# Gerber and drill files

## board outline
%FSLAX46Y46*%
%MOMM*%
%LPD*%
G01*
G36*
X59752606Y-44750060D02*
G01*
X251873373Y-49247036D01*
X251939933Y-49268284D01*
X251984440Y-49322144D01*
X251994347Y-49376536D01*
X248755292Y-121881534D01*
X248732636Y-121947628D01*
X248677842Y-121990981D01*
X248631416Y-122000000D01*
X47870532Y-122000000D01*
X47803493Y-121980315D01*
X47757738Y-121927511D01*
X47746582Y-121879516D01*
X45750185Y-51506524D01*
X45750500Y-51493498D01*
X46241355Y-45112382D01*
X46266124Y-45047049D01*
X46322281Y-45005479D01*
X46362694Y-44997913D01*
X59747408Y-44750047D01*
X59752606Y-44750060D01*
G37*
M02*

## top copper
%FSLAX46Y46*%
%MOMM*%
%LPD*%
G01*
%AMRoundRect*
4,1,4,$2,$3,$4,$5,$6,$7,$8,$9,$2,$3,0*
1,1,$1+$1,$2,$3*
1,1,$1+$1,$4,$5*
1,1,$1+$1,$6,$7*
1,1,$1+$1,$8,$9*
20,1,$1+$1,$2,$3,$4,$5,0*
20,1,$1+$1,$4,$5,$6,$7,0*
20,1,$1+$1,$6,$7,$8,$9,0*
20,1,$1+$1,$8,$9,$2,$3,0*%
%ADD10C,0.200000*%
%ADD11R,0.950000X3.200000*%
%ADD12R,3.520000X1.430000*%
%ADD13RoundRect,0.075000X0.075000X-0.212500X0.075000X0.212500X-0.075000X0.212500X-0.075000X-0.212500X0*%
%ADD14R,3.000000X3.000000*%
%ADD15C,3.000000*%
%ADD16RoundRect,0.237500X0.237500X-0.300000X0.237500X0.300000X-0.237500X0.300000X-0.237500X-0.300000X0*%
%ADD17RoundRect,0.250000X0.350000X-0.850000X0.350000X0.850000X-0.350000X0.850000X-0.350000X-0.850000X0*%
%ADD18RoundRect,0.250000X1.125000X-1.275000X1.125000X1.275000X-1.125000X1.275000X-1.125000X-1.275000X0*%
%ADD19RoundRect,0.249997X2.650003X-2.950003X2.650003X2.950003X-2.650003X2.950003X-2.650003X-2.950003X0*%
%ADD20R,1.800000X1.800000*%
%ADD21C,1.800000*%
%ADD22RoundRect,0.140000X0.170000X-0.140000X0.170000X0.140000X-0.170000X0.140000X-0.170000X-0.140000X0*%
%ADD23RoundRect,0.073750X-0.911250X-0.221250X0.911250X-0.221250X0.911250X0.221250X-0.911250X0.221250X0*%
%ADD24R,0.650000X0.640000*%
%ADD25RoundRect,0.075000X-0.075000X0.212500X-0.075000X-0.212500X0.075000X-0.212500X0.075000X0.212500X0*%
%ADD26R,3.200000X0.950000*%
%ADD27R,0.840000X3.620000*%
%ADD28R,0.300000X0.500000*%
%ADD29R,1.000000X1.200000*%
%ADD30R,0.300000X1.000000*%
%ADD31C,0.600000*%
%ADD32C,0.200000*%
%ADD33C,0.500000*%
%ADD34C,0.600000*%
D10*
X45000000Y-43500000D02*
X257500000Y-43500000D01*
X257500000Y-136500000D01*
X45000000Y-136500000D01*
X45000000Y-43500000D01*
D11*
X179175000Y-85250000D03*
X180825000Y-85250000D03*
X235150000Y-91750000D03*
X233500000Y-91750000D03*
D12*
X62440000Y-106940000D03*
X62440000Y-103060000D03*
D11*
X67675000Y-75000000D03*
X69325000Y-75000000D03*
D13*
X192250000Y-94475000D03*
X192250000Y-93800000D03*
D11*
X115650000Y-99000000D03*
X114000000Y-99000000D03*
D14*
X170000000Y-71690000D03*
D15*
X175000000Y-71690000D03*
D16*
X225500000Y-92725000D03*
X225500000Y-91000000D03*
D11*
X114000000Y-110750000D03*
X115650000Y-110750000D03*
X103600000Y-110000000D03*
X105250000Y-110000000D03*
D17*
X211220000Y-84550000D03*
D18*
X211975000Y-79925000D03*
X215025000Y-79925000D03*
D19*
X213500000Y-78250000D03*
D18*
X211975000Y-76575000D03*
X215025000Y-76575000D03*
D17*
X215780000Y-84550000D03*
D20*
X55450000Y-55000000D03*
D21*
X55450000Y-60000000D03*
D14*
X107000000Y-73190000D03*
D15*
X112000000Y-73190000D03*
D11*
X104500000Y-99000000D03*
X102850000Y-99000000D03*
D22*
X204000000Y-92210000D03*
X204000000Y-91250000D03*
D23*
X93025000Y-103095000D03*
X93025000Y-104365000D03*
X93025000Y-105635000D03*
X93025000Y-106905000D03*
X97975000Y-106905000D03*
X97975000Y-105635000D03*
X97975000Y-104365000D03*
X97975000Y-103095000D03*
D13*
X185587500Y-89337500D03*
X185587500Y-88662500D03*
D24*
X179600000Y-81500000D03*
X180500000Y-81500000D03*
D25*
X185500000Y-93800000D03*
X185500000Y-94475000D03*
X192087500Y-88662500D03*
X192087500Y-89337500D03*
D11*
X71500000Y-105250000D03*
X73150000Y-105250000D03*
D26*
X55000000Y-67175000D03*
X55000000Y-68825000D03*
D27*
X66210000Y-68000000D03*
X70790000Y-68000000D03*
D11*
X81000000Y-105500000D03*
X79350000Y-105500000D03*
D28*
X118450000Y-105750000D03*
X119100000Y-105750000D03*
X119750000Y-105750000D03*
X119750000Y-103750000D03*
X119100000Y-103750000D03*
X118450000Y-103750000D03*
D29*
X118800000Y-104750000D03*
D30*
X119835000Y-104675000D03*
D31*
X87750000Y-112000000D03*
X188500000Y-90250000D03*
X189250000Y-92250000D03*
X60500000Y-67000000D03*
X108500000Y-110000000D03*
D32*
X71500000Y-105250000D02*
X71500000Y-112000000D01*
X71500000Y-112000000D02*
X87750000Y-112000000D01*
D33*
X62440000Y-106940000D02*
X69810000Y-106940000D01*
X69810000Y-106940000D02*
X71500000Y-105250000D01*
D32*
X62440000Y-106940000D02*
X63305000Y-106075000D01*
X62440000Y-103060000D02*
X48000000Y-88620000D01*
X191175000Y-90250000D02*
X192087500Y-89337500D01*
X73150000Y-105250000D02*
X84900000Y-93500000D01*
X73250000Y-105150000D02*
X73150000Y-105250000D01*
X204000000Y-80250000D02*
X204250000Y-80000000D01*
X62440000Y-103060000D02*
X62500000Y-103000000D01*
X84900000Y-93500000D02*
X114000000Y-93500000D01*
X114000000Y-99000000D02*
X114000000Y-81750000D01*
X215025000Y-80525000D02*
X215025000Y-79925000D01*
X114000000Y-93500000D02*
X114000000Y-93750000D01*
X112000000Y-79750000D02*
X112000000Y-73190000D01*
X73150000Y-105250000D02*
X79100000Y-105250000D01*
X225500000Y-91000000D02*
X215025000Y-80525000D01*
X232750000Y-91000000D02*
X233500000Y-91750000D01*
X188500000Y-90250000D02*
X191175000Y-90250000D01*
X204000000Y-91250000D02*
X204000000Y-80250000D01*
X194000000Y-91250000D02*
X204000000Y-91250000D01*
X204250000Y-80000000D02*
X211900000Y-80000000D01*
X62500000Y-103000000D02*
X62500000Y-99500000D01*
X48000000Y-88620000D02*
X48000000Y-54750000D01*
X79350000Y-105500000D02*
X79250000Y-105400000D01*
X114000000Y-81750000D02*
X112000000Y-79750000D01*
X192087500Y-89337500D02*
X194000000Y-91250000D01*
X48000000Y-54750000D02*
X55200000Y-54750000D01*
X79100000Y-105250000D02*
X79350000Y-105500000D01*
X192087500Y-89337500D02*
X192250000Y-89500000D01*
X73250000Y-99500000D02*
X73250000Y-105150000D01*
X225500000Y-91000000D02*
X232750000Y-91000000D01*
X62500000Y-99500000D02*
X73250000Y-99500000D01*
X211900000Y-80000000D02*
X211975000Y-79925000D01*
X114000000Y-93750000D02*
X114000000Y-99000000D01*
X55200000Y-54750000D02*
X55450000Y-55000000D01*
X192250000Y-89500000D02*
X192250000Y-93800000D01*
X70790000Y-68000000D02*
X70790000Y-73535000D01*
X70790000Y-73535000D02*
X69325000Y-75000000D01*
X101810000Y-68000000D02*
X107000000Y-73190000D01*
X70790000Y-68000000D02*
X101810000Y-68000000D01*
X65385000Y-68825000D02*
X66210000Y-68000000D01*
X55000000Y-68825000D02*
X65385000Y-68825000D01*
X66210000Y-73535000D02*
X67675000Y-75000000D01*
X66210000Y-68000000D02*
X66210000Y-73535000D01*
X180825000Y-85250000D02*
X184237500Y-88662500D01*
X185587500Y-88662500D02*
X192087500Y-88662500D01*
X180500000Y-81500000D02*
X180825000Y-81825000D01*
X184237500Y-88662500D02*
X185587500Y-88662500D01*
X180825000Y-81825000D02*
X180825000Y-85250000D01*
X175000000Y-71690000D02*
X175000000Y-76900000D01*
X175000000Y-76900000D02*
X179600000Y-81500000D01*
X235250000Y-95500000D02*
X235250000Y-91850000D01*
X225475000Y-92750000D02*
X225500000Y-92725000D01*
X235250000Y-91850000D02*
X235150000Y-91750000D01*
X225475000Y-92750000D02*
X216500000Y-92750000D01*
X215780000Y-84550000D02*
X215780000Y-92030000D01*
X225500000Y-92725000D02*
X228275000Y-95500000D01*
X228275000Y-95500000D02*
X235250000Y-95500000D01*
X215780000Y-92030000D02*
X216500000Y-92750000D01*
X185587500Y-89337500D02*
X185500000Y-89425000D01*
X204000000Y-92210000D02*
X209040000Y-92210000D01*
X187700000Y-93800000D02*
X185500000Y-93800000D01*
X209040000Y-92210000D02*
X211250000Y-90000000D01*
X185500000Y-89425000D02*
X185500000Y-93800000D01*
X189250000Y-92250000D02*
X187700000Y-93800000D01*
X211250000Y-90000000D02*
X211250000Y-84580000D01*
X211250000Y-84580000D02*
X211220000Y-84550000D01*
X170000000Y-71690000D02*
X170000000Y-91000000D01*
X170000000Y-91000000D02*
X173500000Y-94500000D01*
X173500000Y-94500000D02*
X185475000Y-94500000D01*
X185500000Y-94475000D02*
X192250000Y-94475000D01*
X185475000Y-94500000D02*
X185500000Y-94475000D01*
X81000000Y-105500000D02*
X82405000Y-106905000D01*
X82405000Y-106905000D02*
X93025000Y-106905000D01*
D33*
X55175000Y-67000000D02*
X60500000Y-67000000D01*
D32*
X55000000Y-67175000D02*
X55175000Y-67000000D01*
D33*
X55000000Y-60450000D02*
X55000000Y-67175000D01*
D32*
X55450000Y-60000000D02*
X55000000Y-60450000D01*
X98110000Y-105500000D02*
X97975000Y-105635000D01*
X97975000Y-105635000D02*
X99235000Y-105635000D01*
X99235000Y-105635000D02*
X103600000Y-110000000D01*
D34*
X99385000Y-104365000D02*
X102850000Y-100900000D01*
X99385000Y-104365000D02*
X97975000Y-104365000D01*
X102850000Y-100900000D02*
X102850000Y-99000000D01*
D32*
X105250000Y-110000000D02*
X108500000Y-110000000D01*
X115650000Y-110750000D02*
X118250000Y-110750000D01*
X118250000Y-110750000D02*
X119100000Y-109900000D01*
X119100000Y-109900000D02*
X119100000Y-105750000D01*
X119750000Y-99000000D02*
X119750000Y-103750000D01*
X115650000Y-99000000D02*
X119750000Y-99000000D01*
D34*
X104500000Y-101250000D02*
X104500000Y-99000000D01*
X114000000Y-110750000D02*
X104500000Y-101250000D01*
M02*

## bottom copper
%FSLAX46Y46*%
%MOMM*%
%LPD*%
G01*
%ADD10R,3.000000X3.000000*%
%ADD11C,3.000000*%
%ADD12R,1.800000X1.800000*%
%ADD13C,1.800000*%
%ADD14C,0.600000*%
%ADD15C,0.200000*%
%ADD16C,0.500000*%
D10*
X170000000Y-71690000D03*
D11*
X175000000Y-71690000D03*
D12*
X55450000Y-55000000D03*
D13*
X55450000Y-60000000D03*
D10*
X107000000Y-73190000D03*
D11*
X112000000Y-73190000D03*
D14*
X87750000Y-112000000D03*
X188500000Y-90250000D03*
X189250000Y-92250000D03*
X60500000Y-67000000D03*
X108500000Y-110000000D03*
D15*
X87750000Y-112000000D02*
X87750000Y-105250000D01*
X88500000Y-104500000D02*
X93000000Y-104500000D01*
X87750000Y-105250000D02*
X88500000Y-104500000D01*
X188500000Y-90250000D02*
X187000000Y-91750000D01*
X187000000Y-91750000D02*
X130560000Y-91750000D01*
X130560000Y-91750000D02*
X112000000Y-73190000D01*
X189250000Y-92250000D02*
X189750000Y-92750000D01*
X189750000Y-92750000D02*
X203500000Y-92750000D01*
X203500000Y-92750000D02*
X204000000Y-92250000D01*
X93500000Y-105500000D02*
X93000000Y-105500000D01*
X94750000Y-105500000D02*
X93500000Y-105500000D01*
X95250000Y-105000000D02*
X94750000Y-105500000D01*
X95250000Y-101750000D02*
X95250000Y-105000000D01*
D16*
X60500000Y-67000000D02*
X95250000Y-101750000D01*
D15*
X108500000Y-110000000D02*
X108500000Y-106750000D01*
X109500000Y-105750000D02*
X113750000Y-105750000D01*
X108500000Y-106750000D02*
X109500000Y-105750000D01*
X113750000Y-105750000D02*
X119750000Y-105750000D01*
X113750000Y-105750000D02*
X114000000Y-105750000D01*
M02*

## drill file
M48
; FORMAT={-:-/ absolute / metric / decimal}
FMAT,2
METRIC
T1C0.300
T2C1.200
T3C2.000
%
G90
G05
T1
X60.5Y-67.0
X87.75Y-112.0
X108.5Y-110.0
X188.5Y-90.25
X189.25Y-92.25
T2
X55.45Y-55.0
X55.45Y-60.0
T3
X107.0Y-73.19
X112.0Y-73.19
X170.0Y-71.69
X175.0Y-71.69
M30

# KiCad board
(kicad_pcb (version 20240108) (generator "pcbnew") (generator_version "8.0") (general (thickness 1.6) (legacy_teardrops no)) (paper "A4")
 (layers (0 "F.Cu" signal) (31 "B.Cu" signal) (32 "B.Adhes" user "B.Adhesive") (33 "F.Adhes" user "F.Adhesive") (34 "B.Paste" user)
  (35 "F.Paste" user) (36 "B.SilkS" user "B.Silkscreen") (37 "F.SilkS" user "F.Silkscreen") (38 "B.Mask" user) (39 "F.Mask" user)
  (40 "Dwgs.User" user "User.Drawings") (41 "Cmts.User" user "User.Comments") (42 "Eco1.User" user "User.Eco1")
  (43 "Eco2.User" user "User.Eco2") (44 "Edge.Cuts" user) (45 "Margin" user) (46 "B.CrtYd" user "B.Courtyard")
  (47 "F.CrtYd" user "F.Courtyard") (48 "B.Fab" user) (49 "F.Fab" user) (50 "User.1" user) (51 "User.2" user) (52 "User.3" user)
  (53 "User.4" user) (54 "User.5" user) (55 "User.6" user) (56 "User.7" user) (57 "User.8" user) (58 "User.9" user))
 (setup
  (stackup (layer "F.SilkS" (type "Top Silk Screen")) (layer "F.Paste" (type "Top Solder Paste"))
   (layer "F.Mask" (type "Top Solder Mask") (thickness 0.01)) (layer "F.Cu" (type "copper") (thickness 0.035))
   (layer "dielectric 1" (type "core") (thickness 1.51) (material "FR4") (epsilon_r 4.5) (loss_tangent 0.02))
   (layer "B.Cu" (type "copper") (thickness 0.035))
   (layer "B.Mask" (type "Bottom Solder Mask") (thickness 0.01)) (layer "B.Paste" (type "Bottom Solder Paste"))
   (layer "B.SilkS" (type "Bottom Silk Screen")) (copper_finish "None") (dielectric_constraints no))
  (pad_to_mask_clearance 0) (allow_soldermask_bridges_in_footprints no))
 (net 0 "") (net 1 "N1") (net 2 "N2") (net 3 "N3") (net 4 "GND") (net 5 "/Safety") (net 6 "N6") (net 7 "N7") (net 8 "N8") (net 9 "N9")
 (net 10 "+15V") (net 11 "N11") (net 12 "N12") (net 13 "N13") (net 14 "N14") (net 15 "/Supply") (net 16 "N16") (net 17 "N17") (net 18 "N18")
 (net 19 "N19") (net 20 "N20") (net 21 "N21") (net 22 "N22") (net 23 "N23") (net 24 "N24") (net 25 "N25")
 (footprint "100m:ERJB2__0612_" (layer "F.Cu") (at 180 85.25)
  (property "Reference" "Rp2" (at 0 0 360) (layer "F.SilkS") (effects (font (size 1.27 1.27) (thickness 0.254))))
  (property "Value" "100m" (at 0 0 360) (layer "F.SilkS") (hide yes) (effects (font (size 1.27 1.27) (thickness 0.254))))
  (pad "1" smd rect (at -0.825 0) (size 0.95 3.2) (layers "F.Cu" "F.Paste" "F.Mask") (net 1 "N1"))
  (pad "2" smd rect (at 0.825 0) (size 0.95 3.2) (layers "F.Cu" "F.Paste" "F.Mask") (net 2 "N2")))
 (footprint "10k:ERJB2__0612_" (layer "F.Cu") (at 234.325 91.75 180)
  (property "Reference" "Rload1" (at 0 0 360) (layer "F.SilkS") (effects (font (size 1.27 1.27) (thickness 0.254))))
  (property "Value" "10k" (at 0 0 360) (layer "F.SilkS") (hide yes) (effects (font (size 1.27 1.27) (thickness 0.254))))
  (pad "1" smd rect (at -0.825 0 180) (size 0.95 3.2) (layers "F.Cu" "F.Paste" "F.Mask") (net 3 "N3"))
  (pad "2" smd rect (at 0.825 0 180) (size 0.95 3.2) (layers "F.Cu" "F.Paste" "F.Mask") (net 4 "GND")))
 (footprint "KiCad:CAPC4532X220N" (layer "F.Cu") (at 62.44 105 90)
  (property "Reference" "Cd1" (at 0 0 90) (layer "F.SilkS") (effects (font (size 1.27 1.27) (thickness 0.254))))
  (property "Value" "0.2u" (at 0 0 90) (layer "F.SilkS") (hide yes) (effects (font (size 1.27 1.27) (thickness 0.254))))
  (pad "1" smd rect (at -1.94 0 90) (size 1.43 3.52) (layers "F.Cu" "F.Paste" "F.Mask") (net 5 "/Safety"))
  (pad "2" smd rect (at 1.94 0 90) (size 1.43 3.52) (layers "F.Cu" "F.Paste" "F.Mask") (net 4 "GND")))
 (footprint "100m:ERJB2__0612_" (layer "F.Cu") (at 68.5 75)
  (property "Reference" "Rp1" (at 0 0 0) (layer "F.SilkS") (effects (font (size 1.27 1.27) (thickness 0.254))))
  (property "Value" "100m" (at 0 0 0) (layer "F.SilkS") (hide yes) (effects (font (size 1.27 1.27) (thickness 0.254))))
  (pad "1" smd rect (at -0.825 0) (size 0.95 3.2) (layers "F.Cu" "F.Paste" "F.Mask") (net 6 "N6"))
  (pad "2" smd rect (at 0.825 0) (size 0.95 3.2) (layers "F.Cu" "F.Paste" "F.Mask") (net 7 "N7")))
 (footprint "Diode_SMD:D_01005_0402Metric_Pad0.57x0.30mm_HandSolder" (layer "F.Cu") (at 192.25 94.1375 90)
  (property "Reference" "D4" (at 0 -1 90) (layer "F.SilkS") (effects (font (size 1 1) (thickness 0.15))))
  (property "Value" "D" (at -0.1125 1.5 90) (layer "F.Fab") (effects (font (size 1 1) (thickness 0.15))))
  (pad "" smd roundrect (at -0.3625 0 90) (size 0.41 0.27) (layers "F.Paste") (roundrect_rratio 0.25))
  (pad "" smd roundrect (at 0.3625 0 90) (size 0.41 0.27) (layers "F.Paste") (roundrect_rratio 0.25))
  (pad "1" smd roundrect (at -0.3375 0 90) (size 0.575 0.3) (layers "F.Cu" "F.Mask") (roundrect_rratio 0.25) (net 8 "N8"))
  (pad "2" smd roundrect (at 0.3375 0 90) (size 0.575 0.3) (layers "F.Cu" "F.Mask") (roundrect_rratio 0.25) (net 4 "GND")))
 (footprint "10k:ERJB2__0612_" (layer "F.Cu") (at 114.825 99 180)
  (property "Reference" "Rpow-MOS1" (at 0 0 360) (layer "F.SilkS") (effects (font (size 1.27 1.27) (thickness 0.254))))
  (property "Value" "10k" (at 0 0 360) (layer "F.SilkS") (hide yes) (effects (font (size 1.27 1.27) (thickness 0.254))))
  (pad "1" smd rect (at -0.825 0 180) (size 0.95 3.2) (layers "F.Cu" "F.Paste" "F.Mask") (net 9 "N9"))
  (pad "2" smd rect (at 0.825 0 180) (size 0.95 3.2) (layers "F.Cu" "F.Paste" "F.Mask") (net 4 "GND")))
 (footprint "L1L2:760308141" (layer "F.Cu") (at 170 71.69)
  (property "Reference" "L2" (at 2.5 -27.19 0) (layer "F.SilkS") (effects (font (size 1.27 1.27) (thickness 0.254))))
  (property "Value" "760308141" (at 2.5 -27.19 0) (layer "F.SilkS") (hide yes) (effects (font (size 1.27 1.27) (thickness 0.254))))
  (pad "1" thru_hole rect (at 0 0) (size 3 3) (drill 2) (layers "*.Cu" "*.Mask") (remove_unused_layers no) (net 8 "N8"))
  (pad "2" thru_hole circle (at 5 0) (size 3 3) (drill 2) (layers "*.Cu" "*.Mask") (remove_unused_layers no) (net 1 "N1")))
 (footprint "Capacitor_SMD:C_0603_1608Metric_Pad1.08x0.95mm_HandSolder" (layer "F.Cu") (at 225.5 91.8625 90)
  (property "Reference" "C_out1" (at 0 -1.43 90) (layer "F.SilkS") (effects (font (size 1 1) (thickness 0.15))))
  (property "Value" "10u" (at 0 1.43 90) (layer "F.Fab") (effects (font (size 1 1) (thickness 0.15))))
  (pad "1" smd roundrect (at -0.8625 0 90) (size 1.075 0.95) (layers "F.Cu" "F.Paste" "F.Mask") (roundrect_rratio 0.25) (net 3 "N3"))
  (pad "2" smd roundrect (at 0.8625 0 90) (size 1.075 0.95) (layers "F.Cu" "F.Paste" "F.Mask") (roundrect_rratio 0.25) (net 4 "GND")))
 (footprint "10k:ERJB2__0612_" (layer "F.Cu") (at 114.825 110.75)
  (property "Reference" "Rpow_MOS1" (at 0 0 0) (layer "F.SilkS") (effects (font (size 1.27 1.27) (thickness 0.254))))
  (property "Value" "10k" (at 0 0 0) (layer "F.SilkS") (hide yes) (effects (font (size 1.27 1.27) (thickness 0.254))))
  (pad "1" smd rect (at -0.825 0) (size 0.95 3.2) (layers "F.Cu" "F.Paste" "F.Mask") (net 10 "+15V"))
  (pad "2" smd rect (at 0.825 0) (size 0.95 3.2) (layers "F.Cu" "F.Paste" "F.Mask") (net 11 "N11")))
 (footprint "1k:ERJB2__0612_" (layer "F.Cu") (at 104.425 110)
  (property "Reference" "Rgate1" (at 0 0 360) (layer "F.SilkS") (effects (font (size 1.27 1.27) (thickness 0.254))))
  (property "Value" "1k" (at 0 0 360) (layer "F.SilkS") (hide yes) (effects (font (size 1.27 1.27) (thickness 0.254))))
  (pad "1" smd rect (at -0.825 0) (size 0.95 3.2) (layers "F.Cu" "F.Paste" "F.Mask") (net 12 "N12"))
  (pad "2" smd rect (at 0.825 0) (size 0.95 3.2) (layers "F.Cu" "F.Paste" "F.Mask") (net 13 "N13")))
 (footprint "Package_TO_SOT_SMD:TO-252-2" (layer "F.Cu") (at 213.5 79.51 90)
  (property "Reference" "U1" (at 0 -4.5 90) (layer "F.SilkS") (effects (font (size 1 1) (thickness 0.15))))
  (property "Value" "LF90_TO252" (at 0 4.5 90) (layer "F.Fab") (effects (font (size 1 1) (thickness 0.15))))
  (pad "1" smd roundrect (at -5.04 -2.28 90) (size 2.2 1.2) (layers "F.Cu" "F.Paste" "F.Mask") (roundrect_rratio 0.208333) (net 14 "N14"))
  (pad "2" smd roundrect (at -0.415 -1.525 90) (size 3.05 2.75) (layers "F.Cu" "F.Paste") (roundrect_rratio 0.090909) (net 4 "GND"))
  (pad "2" smd roundrect (at -0.415 1.525 90) (size 3.05 2.75) (layers "F.Cu" "F.Paste") (roundrect_rratio 0.090909) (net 4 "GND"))
  (pad "2" smd roundrect (at 1.26 0 90) (size 6.4 5.8) (layers "F.Cu" "F.Mask") (roundrect_rratio 0.043103) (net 4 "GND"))
  (pad "2" smd roundrect (at 2.935 -1.525 90) (size 3.05 2.75) (layers "F.Cu" "F.Paste") (roundrect_rratio 0.090909) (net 4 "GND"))
  (pad "2" smd roundrect (at 2.935 1.525 90) (size 3.05 2.75) (layers "F.Cu" "F.Paste") (roundrect_rratio 0.090909) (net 4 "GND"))
  (pad "3" smd roundrect (at -5.04 2.28 90) (size 2.2 1.2) (layers "F.Cu" "F.Paste" "F.Mask") (roundrect_rratio 0.208333) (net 3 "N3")))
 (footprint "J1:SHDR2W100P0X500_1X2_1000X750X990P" (layer "F.Cu") (at 55.45 55 -90)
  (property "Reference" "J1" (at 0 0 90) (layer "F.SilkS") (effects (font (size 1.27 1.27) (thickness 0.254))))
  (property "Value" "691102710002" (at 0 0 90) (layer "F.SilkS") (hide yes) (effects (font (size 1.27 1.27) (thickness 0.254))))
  (pad "1" thru_hole rect (at 0 0 270) (size 1.8 1.8) (drill 1.2) (layers "*.Cu" "*.Mask") (remove_unused_layers no) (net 4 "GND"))
  (pad "2" thru_hole circle (at 5 0 270) (size 1.8 1.8) (drill 1.2) (layers "*.Cu" "*.Mask") (remove_unused_layers no) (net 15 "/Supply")))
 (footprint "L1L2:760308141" (layer "F.Cu") (at 107 73.19)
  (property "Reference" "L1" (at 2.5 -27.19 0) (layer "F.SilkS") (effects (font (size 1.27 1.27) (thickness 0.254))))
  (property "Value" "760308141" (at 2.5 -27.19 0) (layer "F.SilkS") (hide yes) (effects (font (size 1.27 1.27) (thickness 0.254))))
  (pad "1" thru_hole rect (at 0 0) (size 3 3) (drill 2) (layers "*.Cu" "*.Mask") (remove_unused_layers no) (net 7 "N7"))
  (pad "2" thru_hole circle (at 5 0) (size 3 3) (drill 2) (layers "*.Cu" "*.Mask") (remove_unused_layers no) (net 4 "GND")))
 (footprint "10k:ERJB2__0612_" (layer "F.Cu") (at 103.675 99 180)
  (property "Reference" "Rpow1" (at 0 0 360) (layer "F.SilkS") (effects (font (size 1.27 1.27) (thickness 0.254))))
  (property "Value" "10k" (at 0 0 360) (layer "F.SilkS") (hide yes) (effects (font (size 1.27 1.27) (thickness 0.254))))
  (pad "1" smd rect (at -0.825 0 180) (size 0.95 3.2) (layers "F.Cu" "F.Paste" "F.Mask") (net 10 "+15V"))
  (pad "2" smd rect (at 0.825 0 180) (size 0.95 3.2) (layers "F.Cu" "F.Paste" "F.Mask") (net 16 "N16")))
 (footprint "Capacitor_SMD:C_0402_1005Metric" (layer "F.Cu") (at 204 91.73 90)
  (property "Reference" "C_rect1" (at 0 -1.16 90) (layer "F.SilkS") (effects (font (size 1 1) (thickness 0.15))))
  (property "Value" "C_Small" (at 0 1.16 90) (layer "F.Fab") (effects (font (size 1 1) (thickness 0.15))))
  (pad "1" smd roundrect (at -0.48 0 90) (size 0.56 0.62) (layers "F.Cu" "F.Paste" "F.Mask") (roundrect_rratio 0.25) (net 14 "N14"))
  (pad "2" smd roundrect (at 0.48 0 90) (size 0.56 0.62) (layers "F.Cu" "F.Paste" "F.Mask") (roundrect_rratio 0.25) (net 4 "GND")))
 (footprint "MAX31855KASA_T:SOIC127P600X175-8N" (layer "F.Cu") (at 95.5 105)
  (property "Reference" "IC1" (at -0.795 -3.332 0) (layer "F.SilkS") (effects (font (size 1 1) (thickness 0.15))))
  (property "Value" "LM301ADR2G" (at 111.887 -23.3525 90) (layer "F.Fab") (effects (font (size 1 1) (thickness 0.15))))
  (pad "1" smd roundrect (at -2.475 -1.905) (size 1.97 0.59) (layers "F.Cu" "F.Paste" "F.Mask") (roundrect_rratio 0.125) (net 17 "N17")
   (solder_mask_margin 0.102))
  (pad "2" smd roundrect (at -2.475 -0.635) (size 1.97 0.59) (layers "F.Cu" "F.Paste" "F.Mask") (roundrect_rratio 0.125) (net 5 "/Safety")
   (solder_mask_margin 0.102))
  (pad "3" smd roundrect (at -2.475 0.635) (size 1.97 0.59) (layers "F.Cu" "F.Paste" "F.Mask") (roundrect_rratio 0.125) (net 15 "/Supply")
   (solder_mask_margin 0.102))
  (pad "4" smd roundrect (at -2.475 1.905) (size 1.97 0.59) (layers "F.Cu" "F.Paste" "F.Mask") (roundrect_rratio 0.125) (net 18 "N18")
   (solder_mask_margin 0.102))
  (pad "5" smd roundrect (at 2.475 1.905) (size 1.97 0.59) (layers "F.Cu" "F.Paste" "F.Mask") (roundrect_rratio 0.125) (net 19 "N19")
   (solder_mask_margin 0.102))
  (pad "6" smd roundrect (at 2.475 0.635) (size 1.97 0.59) (layers "F.Cu" "F.Paste" "F.Mask") (roundrect_rratio 0.125) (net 12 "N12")
   (solder_mask_margin 0.102))
  (pad "7" smd roundrect (at 2.475 -0.635) (size 1.97 0.59) (layers "F.Cu" "F.Paste" "F.Mask") (roundrect_rratio 0.125) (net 16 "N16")
   (solder_mask_margin 0.102))
  (pad "8" smd roundrect (at 2.475 -1.905) (size 1.97 0.59) (layers "F.Cu" "F.Paste" "F.Mask") (roundrect_rratio 0.125) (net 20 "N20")
   (solder_mask_margin 0.102)))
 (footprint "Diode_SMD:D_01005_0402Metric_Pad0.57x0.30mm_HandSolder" (layer "F.Cu") (at 185.5875 89 90)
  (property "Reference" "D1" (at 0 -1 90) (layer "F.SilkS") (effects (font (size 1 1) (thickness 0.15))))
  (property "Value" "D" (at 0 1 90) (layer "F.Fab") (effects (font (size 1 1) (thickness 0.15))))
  (pad "" smd roundrect (at -0.3625 0 90) (size 0.41 0.27) (layers "F.Paste") (roundrect_rratio 0.25))
  (pad "" smd roundrect (at 0.3625 0 90) (size 0.41 0.27) (layers "F.Paste") (roundrect_rratio 0.25))
  (pad "1" smd roundrect (at -0.3375 0 90) (size 0.575 0.3) (layers "F.Cu" "F.Mask") (roundrect_rratio 0.25) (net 14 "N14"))
  (pad "2" smd roundrect (at 0.3375 0 90) (size 0.575 0.3) (layers "F.Cu" "F.Mask") (roundrect_rratio 0.25) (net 2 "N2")))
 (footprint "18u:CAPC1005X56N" (layer "F.Cu") (at 180.05 81.5)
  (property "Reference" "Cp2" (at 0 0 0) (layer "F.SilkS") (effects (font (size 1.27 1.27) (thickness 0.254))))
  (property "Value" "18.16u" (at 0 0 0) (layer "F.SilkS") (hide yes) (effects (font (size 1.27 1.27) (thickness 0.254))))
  (pad "1" smd rect (at -0.45 0 90) (size 0.64 0.65) (layers "F.Cu" "F.Paste" "F.Mask") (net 1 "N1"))
  (pad "2" smd rect (at 0.45 0 90) (size 0.64 0.65) (layers "F.Cu" "F.Paste" "F.Mask") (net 2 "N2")))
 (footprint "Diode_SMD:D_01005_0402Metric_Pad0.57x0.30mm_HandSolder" (layer "F.Cu") (at 185.5 94.1375 -90)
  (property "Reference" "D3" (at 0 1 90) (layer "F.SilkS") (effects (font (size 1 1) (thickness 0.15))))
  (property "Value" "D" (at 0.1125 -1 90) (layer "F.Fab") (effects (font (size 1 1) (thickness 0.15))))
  (pad "" smd roundrect (at -0.3625 0 270) (size 0.41 0.27) (layers "F.Paste") (roundrect_rratio 0.25))
  (pad "" smd roundrect (at 0.3625 0 270) (size 0.41 0.27) (layers "F.Paste") (roundrect_rratio 0.25))
  (pad "1" smd roundrect (at -0.3375 0 270) (size 0.575 0.3) (layers "F.Cu" "F.Mask") (roundrect_rratio 0.25) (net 14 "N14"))
  (pad "2" smd roundrect (at 0.3375 0 270) (size 0.575 0.3) (layers "F.Cu" "F.Mask") (roundrect_rratio 0.25) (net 8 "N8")))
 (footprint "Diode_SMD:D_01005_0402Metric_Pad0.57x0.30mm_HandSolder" (layer "F.Cu") (at 192.0875 89 -90)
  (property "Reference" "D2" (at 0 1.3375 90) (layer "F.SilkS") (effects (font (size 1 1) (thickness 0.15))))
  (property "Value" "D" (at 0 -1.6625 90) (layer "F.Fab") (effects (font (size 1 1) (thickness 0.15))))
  (pad "" smd roundrect (at -0.3625 0 270) (size 0.41 0.27) (layers "F.Paste") (roundrect_rratio 0.25))
  (pad "" smd roundrect (at 0.3625 0 270) (size 0.41 0.27) (layers "F.Paste") (roundrect_rratio 0.25))
  (pad "1" smd roundrect (at -0.3375 0 270) (size 0.575 0.3) (layers "F.Cu" "F.Mask") (roundrect_rratio 0.25) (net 2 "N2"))
  (pad "2" smd roundrect (at 0.3375 0 270) (size 0.575 0.3) (layers "F.Cu" "F.Mask") (roundrect_rratio 0.25) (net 4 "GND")))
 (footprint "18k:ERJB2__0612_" (layer "F.Cu") (at 72.325 105.25)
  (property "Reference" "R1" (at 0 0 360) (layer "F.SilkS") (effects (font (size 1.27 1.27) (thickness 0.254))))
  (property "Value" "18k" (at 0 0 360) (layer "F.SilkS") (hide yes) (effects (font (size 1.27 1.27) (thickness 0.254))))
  (pad "1" smd rect (at -0.825 0) (size 0.95 3.2) (layers "F.Cu" "F.Paste" "F.Mask") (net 5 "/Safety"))
  (pad "2" smd rect (at 0.825 0) (size 0.95 3.2) (layers "F.Cu" "F.Paste" "F.Mask") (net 4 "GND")))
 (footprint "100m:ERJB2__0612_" (layer "F.Cu") (at 55 68 -90)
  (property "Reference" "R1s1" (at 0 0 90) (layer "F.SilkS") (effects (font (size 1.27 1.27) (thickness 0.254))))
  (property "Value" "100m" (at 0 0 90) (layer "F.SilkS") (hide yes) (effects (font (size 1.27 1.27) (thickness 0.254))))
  (pad "1" smd rect (at -0.825 0 270) (size 0.95 3.2) (layers "F.Cu" "F.Paste" "F.Mask") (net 15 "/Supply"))
  (pad "2" smd rect (at 0.825 0 270) (size 0.95 3.2) (layers "F.Cu" "F.Paste" "F.Mask") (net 6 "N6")))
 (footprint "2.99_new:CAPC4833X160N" (layer "F.Cu") (at 68.5 68)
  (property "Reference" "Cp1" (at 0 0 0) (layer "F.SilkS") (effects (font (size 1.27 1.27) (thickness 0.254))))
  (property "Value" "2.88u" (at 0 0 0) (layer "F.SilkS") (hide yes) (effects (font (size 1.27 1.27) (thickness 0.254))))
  (pad "1" smd rect (at -2.29 0) (size 0.84 3.62) (layers "F.Cu" "F.Paste" "F.Mask") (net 6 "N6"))
  (pad "2" smd rect (at 2.29 0) (size 0.84 3.62) (layers "F.Cu" "F.Paste" "F.Mask") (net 7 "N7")))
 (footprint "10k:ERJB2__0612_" (layer "F.Cu") (at 80.175 105.5 180)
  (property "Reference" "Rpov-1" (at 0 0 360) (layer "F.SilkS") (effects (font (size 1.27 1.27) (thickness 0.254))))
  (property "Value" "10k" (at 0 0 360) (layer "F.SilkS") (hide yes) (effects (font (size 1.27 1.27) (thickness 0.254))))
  (pad "1" smd rect (at -0.825 0 180) (size 0.95 3.2) (layers "F.Cu" "F.Paste" "F.Mask") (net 18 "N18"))
  (pad "2" smd rect (at 0.825 0 180) (size 0.95 3.2) (layers "F.Cu" "F.Paste" "F.Mask") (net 4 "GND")))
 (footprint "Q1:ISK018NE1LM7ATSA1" (layer "F.Cu") (at 119.1 104.75)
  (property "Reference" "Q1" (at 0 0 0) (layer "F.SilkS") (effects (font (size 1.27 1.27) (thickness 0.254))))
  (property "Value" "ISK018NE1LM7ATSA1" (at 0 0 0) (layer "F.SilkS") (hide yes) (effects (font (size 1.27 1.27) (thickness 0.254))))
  (pad "1" smd rect (at -0.65 1) (size 0.3 0.5) (layers "F.Cu" "F.Paste" "F.Mask") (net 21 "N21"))
  (pad "2" smd rect (at 0 1) (size 0.3 0.5) (layers "F.Cu" "F.Paste" "F.Mask") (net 11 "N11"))
  (pad "3" smd rect (at 0.65 1) (size 0.3 0.5) (layers "F.Cu" "F.Paste" "F.Mask") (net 13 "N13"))
  (pad "4" smd rect (at 0.65 -1) (size 0.3 0.5) (layers "F.Cu" "F.Paste" "F.Mask") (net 9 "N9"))
  (pad "5" smd rect (at 0 -1) (size 0.3 0.5) (layers "F.Cu" "F.Paste" "F.Mask") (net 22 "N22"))
  (pad "6" smd rect (at -0.65 -1) (size 0.3 0.5) (layers "F.Cu" "F.Paste" "F.Mask") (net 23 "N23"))
  (pad "7" smd rect (at -0.3 0) (size 1 1.2) (layers "F.Cu" "F.Paste" "F.Mask") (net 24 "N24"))
  (pad "8" smd rect (at 0.735 -0.075) (size 0.3 1) (layers "F.Cu" "F.Paste" "F.Mask") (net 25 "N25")))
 (gr_rect (start 45 43.5) (end 257.5 136.5) (stroke (width 0.2) (type default)) (fill none) (layer "F.Cu"))
 (segment (start 71.5 105.25) (end 71.5 112) (width 0.2) (layer "F.Cu") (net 5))
 (segment (start 71.5 112) (end 87.75 112) (width 0.2) (layer "F.Cu") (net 5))
 (segment (start 62.44 106.94) (end 69.81 106.94) (width 0.5) (layer "F.Cu") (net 5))
 (segment (start 69.81 106.94) (end 71.5 105.25) (width 0.5) (layer "F.Cu") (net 5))
 (segment (start 62.44 106.94) (end 63.305 106.075) (width 0.2) (layer "F.Cu") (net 5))
 (via (at 87.75 112) (size 0.6) (drill 0.3) (layers "F.Cu" "B.Cu") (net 5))
 (segment (start 87.75 112) (end 87.75 105.25) (width 0.2) (layer "B.Cu") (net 5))
 (segment (start 88.5 104.5) (end 93 104.5) (width 0.2) (layer "B.Cu") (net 5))
 (segment (start 87.75 105.25) (end 88.5 104.5) (width 0.2) (layer "B.Cu") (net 5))
 (segment (start 62.44 103.06) (end 48 88.62) (width 0.2) (layer "F.Cu") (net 4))
 (segment (start 191.175 90.25) (end 192.0875 89.3375) (width 0.2) (layer "F.Cu") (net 4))
 (segment (start 73.15 105.25) (end 84.9 93.5) (width 0.2) (layer "F.Cu") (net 4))
 (segment (start 73.25 105.15) (end 73.15 105.25) (width 0.2) (layer "F.Cu") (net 4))
 (segment (start 204 80.25) (end 204.25 80) (width 0.2) (layer "F.Cu") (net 4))
 (segment (start 62.44 103.06) (end 62.5 103) (width 0.2) (layer "F.Cu") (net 4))
 (segment (start 84.9 93.5) (end 114 93.5) (width 0.2) (layer "F.Cu") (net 4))
 (segment (start 114 99) (end 114 81.75) (width 0.2) (layer "F.Cu") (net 4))
 (segment (start 215.025 80.525) (end 215.025 79.925) (width 0.2) (layer "F.Cu") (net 4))
 (segment (start 114 93.5) (end 114 93.75) (width 0.2) (layer "F.Cu") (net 4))
 (segment (start 112 79.75) (end 112 73.19) (width 0.2) (layer "F.Cu") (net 4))
 (segment (start 73.15 105.25) (end 79.1 105.25) (width 0.2) (layer "F.Cu") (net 4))
 (segment (start 225.5 91) (end 215.025 80.525) (width 0.2) (layer "F.Cu") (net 4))
 (segment (start 232.75 91) (end 233.5 91.75) (width 0.2) (layer "F.Cu") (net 4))
 (segment (start 188.5 90.25) (end 191.175 90.25) (width 0.2) (layer "F.Cu") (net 4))
 (segment (start 204 91.25) (end 204 80.25) (width 0.2) (layer "F.Cu") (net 4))
 (segment (start 194 91.25) (end 204 91.25) (width 0.2) (layer "F.Cu") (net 4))
 (segment (start 204.25 80) (end 211.9 80) (width 0.2) (layer "F.Cu") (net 4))
 (segment (start 62.5 103) (end 62.5 99.5) (width 0.2) (layer "F.Cu") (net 4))
 (segment (start 48 88.62) (end 48 54.75) (width 0.2) (layer "F.Cu") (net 4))
 (segment (start 79.35 105.5) (end 79.25 105.4) (width 0.2) (layer "F.Cu") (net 4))
 (segment (start 114 81.75) (end 112 79.75) (width 0.2) (layer "F.Cu") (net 4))
 (segment (start 192.0875 89.3375) (end 194 91.25) (width 0.2) (layer "F.Cu") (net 4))
 (segment (start 48 54.75) (end 55.2 54.75) (width 0.2) (layer "F.Cu") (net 4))
 (segment (start 79.1 105.25) (end 79.35 105.5) (width 0.2) (layer "F.Cu") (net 4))
 (segment (start 192.0875 89.3375) (end 192.25 89.5) (width 0.2) (layer "F.Cu") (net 4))
 (segment (start 73.25 99.5) (end 73.25 105.15) (width 0.2) (layer "F.Cu") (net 4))
 (segment (start 225.5 91) (end 232.75 91) (width 0.2) (layer "F.Cu") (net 4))
 (segment (start 62.5 99.5) (end 73.25 99.5) (width 0.2) (layer "F.Cu") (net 4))
 (segment (start 211.9 80) (end 211.975 79.925) (width 0.2) (layer "F.Cu") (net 4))
 (segment (start 114 93.75) (end 114 99) (width 0.2) (layer "F.Cu") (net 4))
 (segment (start 55.2 54.75) (end 55.45 55) (width 0.2) (layer "F.Cu") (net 4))
 (segment (start 192.25 89.5) (end 192.25 93.8) (width 0.2) (layer "F.Cu") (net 4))
 (via (at 188.5 90.25) (size 0.6) (drill 0.3) (layers "F.Cu" "B.Cu") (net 4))
 (segment (start 188.5 90.25) (end 187 91.75) (width 0.2) (layer "B.Cu") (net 4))
 (segment (start 187 91.75) (end 130.56 91.75) (width 0.2) (layer "B.Cu") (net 4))
 (segment (start 130.56 91.75) (end 112 73.19) (width 0.2) (layer "B.Cu") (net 4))
 (segment (start 70.79 68) (end 70.79 73.535) (width 0.2) (layer "F.Cu") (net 7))
 (segment (start 70.79 73.535) (end 69.325 75) (width 0.2) (layer "F.Cu") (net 7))
 (segment (start 101.81 68) (end 107 73.19) (width 0.2) (layer "F.Cu") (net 7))
 (segment (start 70.79 68) (end 101.81 68) (width 0.2) (layer "F.Cu") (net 7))
 (segment (start 65.385 68.825) (end 66.21 68) (width 0.2) (layer "F.Cu") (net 6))
 (segment (start 55 68.825) (end 65.385 68.825) (width 0.2) (layer "F.Cu") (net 6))
 (segment (start 66.21 73.535) (end 67.675 75) (width 0.2) (layer "F.Cu") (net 6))
 (segment (start 66.21 68) (end 66.21 73.535) (width 0.2) (layer "F.Cu") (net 6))
 (segment (start 180.825 85.25) (end 184.2375 88.6625) (width 0.2) (layer "F.Cu") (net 2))
 (segment (start 185.5875 88.6625) (end 192.0875 88.6625) (width 0.2) (layer "F.Cu") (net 2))
 (segment (start 180.5 81.5) (end 180.825 81.825) (width 0.2) (layer "F.Cu") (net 2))
 (segment (start 184.2375 88.6625) (end 185.5875 88.6625) (width 0.2) (layer "F.Cu") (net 2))
 (segment (start 180.825 81.825) (end 180.825 85.25) (width 0.2) (layer "F.Cu") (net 2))
 (segment (start 175 71.69) (end 175 76.9) (width 0.2) (layer "F.Cu") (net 1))
 (segment (start 175 76.9) (end 179.6 81.5) (width 0.2) (layer "F.Cu") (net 1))
 (segment (start 235.25 95.5) (end 235.25 91.85) (width 0.2) (layer "F.Cu") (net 3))
 (segment (start 225.475 92.75) (end 225.5 92.725) (width 0.2) (layer "F.Cu") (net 3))
 (segment (start 235.25 91.85) (end 235.15 91.75) (width 0.2) (layer "F.Cu") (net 3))
 (segment (start 225.475 92.75) (end 216.5 92.75) (width 0.2) (layer "F.Cu") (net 3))
 (segment (start 215.78 84.55) (end 215.78 92.03) (width 0.2) (layer "F.Cu") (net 3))
 (segment (start 225.5 92.725) (end 228.275 95.5) (width 0.2) (layer "F.Cu") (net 3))
 (segment (start 228.275 95.5) (end 235.25 95.5) (width 0.2) (layer "F.Cu") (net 3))
 (segment (start 215.78 92.03) (end 216.5 92.75) (width 0.2) (layer "F.Cu") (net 3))
 (segment (start 185.5875 89.3375) (end 185.5 89.425) (width 0.2) (layer "F.Cu") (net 14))
 (segment (start 204 92.21) (end 209.04 92.21) (width 0.2) (layer "F.Cu") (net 14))
 (segment (start 187.7 93.8) (end 185.5 93.8) (width 0.2) (layer "F.Cu") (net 14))
 (segment (start 209.04 92.21) (end 211.25 90) (width 0.2) (layer "F.Cu") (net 14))
 (segment (start 185.5 89.425) (end 185.5 93.8) (width 0.2) (layer "F.Cu") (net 14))
 (segment (start 189.25 92.25) (end 187.7 93.8) (width 0.2) (layer "F.Cu") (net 14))
 (segment (start 211.25 90) (end 211.25 84.58) (width 0.2) (layer "F.Cu") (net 14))
 (segment (start 211.25 84.58) (end 211.22 84.55) (width 0.2) (layer "F.Cu") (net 14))
 (via (at 189.25 92.25) (size 0.6) (drill 0.3) (layers "F.Cu" "B.Cu") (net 14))
 (segment (start 189.25 92.25) (end 189.75 92.75) (width 0.2) (layer "B.Cu") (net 14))
 (segment (start 189.75 92.75) (end 203.5 92.75) (width 0.2) (layer "B.Cu") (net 14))
 (segment (start 203.5 92.75) (end 204 92.25) (width 0.2) (layer "B.Cu") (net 14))
 (segment (start 170 71.69) (end 170 91) (width 0.2) (layer "F.Cu") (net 8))
 (segment (start 170 91) (end 173.5 94.5) (width 0.2) (layer "F.Cu") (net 8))
 (segment (start 173.5 94.5) (end 185.475 94.5) (width 0.2) (layer "F.Cu") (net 8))
 (segment (start 185.5 94.475) (end 192.25 94.475) (width 0.2) (layer "F.Cu") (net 8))
 (segment (start 185.475 94.5) (end 185.5 94.475) (width 0.2) (layer "F.Cu") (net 8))
 (segment (start 81 105.5) (end 82.405 106.905) (width 0.2) (layer "F.Cu") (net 18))
 (segment (start 82.405 106.905) (end 93.025 106.905) (width 0.2) (layer "F.Cu") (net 18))
 (segment (start 55.175 67) (end 60.5 67) (width 0.5) (layer "F.Cu") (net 15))
 (segment (start 55 67.175) (end 55.175 67) (width 0.2) (layer "F.Cu") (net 15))
 (segment (start 55 60.45) (end 55 67.175) (width 0.5) (layer "F.Cu") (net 15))
 (segment (start 55.45 60) (end 55 60.45) (width 0.2) (layer "F.Cu") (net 15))
 (via (at 60.5 67) (size 0.6) (drill 0.3) (layers "F.Cu" "B.Cu") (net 15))
 (segment (start 93.5 105.5) (end 93 105.5) (width 0.2) (layer "B.Cu") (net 15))
 (segment (start 94.75 105.5) (end 93.5 105.5) (width 0.2) (layer "B.Cu") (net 15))
 (segment (start 95.25 105) (end 94.75 105.5) (width 0.2) (layer "B.Cu") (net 15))
 (segment (start 95.25 101.75) (end 95.25 105) (width 0.2) (layer "B.Cu") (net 15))
 (segment (start 60.5 67) (end 95.25 101.75) (width 0.5) (layer "B.Cu") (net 15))
 (segment (start 98.11 105.5) (end 97.975 105.635) (width 0.2) (layer "F.Cu") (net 12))
 (segment (start 97.975 105.635) (end 99.235 105.635) (width 0.2) (layer "F.Cu") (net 12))
 (segment (start 99.235 105.635) (end 103.6 110) (width 0.2) (layer "F.Cu") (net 12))
 (segment (start 99.385 104.365) (end 102.85 100.9) (width 0.6) (layer "F.Cu") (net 16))
 (segment (start 99.385 104.365) (end 97.975 104.365) (width 0.6) (layer "F.Cu") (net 16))
 (segment (start 102.85 100.9) (end 102.85 99) (width 0.6) (layer "F.Cu") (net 16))
 (segment (start 105.25 110) (end 108.5 110) (width 0.2) (layer "F.Cu") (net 13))
 (via (at 108.5 110) (size 0.6) (drill 0.3) (layers "F.Cu" "B.Cu") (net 13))
 (segment (start 108.5 110) (end 108.5 106.75) (width 0.2) (layer "B.Cu") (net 13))
 (segment (start 109.5 105.75) (end 113.75 105.75) (width 0.2) (layer "B.Cu") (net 13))
 (segment (start 108.5 106.75) (end 109.5 105.75) (width 0.2) (layer "B.Cu") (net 13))
 (segment (start 113.75 105.75) (end 119.75 105.75) (width 0.2) (layer "B.Cu") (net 13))
 (segment (start 113.75 105.75) (end 114 105.75) (width 0.2) (layer "B.Cu") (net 13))
 (segment (start 115.65 110.75) (end 118.25 110.75) (width 0.2) (layer "F.Cu") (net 11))
 (segment (start 118.25 110.75) (end 119.1 109.9) (width 0.2) (layer "F.Cu") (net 11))
 (segment (start 119.1 109.9) (end 119.1 105.75) (width 0.2) (layer "F.Cu") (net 11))
 (segment (start 119.75 99) (end 119.75 103.75) (width 0.2) (layer "F.Cu") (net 9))
 (segment (start 115.65 99) (end 119.75 99) (width 0.2) (layer "F.Cu") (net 9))
 (segment (start 104.5 101.25) (end 104.5 99) (width 0.6) (layer "F.Cu") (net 10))
 (segment (start 114 110.75) (end 104.5 101.25) (width 0.6) (layer "F.Cu") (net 10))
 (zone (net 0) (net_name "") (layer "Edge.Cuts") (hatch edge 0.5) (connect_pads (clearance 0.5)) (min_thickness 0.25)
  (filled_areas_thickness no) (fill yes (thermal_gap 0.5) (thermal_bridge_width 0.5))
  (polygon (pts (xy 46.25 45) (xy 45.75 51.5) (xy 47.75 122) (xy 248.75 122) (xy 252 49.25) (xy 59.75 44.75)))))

